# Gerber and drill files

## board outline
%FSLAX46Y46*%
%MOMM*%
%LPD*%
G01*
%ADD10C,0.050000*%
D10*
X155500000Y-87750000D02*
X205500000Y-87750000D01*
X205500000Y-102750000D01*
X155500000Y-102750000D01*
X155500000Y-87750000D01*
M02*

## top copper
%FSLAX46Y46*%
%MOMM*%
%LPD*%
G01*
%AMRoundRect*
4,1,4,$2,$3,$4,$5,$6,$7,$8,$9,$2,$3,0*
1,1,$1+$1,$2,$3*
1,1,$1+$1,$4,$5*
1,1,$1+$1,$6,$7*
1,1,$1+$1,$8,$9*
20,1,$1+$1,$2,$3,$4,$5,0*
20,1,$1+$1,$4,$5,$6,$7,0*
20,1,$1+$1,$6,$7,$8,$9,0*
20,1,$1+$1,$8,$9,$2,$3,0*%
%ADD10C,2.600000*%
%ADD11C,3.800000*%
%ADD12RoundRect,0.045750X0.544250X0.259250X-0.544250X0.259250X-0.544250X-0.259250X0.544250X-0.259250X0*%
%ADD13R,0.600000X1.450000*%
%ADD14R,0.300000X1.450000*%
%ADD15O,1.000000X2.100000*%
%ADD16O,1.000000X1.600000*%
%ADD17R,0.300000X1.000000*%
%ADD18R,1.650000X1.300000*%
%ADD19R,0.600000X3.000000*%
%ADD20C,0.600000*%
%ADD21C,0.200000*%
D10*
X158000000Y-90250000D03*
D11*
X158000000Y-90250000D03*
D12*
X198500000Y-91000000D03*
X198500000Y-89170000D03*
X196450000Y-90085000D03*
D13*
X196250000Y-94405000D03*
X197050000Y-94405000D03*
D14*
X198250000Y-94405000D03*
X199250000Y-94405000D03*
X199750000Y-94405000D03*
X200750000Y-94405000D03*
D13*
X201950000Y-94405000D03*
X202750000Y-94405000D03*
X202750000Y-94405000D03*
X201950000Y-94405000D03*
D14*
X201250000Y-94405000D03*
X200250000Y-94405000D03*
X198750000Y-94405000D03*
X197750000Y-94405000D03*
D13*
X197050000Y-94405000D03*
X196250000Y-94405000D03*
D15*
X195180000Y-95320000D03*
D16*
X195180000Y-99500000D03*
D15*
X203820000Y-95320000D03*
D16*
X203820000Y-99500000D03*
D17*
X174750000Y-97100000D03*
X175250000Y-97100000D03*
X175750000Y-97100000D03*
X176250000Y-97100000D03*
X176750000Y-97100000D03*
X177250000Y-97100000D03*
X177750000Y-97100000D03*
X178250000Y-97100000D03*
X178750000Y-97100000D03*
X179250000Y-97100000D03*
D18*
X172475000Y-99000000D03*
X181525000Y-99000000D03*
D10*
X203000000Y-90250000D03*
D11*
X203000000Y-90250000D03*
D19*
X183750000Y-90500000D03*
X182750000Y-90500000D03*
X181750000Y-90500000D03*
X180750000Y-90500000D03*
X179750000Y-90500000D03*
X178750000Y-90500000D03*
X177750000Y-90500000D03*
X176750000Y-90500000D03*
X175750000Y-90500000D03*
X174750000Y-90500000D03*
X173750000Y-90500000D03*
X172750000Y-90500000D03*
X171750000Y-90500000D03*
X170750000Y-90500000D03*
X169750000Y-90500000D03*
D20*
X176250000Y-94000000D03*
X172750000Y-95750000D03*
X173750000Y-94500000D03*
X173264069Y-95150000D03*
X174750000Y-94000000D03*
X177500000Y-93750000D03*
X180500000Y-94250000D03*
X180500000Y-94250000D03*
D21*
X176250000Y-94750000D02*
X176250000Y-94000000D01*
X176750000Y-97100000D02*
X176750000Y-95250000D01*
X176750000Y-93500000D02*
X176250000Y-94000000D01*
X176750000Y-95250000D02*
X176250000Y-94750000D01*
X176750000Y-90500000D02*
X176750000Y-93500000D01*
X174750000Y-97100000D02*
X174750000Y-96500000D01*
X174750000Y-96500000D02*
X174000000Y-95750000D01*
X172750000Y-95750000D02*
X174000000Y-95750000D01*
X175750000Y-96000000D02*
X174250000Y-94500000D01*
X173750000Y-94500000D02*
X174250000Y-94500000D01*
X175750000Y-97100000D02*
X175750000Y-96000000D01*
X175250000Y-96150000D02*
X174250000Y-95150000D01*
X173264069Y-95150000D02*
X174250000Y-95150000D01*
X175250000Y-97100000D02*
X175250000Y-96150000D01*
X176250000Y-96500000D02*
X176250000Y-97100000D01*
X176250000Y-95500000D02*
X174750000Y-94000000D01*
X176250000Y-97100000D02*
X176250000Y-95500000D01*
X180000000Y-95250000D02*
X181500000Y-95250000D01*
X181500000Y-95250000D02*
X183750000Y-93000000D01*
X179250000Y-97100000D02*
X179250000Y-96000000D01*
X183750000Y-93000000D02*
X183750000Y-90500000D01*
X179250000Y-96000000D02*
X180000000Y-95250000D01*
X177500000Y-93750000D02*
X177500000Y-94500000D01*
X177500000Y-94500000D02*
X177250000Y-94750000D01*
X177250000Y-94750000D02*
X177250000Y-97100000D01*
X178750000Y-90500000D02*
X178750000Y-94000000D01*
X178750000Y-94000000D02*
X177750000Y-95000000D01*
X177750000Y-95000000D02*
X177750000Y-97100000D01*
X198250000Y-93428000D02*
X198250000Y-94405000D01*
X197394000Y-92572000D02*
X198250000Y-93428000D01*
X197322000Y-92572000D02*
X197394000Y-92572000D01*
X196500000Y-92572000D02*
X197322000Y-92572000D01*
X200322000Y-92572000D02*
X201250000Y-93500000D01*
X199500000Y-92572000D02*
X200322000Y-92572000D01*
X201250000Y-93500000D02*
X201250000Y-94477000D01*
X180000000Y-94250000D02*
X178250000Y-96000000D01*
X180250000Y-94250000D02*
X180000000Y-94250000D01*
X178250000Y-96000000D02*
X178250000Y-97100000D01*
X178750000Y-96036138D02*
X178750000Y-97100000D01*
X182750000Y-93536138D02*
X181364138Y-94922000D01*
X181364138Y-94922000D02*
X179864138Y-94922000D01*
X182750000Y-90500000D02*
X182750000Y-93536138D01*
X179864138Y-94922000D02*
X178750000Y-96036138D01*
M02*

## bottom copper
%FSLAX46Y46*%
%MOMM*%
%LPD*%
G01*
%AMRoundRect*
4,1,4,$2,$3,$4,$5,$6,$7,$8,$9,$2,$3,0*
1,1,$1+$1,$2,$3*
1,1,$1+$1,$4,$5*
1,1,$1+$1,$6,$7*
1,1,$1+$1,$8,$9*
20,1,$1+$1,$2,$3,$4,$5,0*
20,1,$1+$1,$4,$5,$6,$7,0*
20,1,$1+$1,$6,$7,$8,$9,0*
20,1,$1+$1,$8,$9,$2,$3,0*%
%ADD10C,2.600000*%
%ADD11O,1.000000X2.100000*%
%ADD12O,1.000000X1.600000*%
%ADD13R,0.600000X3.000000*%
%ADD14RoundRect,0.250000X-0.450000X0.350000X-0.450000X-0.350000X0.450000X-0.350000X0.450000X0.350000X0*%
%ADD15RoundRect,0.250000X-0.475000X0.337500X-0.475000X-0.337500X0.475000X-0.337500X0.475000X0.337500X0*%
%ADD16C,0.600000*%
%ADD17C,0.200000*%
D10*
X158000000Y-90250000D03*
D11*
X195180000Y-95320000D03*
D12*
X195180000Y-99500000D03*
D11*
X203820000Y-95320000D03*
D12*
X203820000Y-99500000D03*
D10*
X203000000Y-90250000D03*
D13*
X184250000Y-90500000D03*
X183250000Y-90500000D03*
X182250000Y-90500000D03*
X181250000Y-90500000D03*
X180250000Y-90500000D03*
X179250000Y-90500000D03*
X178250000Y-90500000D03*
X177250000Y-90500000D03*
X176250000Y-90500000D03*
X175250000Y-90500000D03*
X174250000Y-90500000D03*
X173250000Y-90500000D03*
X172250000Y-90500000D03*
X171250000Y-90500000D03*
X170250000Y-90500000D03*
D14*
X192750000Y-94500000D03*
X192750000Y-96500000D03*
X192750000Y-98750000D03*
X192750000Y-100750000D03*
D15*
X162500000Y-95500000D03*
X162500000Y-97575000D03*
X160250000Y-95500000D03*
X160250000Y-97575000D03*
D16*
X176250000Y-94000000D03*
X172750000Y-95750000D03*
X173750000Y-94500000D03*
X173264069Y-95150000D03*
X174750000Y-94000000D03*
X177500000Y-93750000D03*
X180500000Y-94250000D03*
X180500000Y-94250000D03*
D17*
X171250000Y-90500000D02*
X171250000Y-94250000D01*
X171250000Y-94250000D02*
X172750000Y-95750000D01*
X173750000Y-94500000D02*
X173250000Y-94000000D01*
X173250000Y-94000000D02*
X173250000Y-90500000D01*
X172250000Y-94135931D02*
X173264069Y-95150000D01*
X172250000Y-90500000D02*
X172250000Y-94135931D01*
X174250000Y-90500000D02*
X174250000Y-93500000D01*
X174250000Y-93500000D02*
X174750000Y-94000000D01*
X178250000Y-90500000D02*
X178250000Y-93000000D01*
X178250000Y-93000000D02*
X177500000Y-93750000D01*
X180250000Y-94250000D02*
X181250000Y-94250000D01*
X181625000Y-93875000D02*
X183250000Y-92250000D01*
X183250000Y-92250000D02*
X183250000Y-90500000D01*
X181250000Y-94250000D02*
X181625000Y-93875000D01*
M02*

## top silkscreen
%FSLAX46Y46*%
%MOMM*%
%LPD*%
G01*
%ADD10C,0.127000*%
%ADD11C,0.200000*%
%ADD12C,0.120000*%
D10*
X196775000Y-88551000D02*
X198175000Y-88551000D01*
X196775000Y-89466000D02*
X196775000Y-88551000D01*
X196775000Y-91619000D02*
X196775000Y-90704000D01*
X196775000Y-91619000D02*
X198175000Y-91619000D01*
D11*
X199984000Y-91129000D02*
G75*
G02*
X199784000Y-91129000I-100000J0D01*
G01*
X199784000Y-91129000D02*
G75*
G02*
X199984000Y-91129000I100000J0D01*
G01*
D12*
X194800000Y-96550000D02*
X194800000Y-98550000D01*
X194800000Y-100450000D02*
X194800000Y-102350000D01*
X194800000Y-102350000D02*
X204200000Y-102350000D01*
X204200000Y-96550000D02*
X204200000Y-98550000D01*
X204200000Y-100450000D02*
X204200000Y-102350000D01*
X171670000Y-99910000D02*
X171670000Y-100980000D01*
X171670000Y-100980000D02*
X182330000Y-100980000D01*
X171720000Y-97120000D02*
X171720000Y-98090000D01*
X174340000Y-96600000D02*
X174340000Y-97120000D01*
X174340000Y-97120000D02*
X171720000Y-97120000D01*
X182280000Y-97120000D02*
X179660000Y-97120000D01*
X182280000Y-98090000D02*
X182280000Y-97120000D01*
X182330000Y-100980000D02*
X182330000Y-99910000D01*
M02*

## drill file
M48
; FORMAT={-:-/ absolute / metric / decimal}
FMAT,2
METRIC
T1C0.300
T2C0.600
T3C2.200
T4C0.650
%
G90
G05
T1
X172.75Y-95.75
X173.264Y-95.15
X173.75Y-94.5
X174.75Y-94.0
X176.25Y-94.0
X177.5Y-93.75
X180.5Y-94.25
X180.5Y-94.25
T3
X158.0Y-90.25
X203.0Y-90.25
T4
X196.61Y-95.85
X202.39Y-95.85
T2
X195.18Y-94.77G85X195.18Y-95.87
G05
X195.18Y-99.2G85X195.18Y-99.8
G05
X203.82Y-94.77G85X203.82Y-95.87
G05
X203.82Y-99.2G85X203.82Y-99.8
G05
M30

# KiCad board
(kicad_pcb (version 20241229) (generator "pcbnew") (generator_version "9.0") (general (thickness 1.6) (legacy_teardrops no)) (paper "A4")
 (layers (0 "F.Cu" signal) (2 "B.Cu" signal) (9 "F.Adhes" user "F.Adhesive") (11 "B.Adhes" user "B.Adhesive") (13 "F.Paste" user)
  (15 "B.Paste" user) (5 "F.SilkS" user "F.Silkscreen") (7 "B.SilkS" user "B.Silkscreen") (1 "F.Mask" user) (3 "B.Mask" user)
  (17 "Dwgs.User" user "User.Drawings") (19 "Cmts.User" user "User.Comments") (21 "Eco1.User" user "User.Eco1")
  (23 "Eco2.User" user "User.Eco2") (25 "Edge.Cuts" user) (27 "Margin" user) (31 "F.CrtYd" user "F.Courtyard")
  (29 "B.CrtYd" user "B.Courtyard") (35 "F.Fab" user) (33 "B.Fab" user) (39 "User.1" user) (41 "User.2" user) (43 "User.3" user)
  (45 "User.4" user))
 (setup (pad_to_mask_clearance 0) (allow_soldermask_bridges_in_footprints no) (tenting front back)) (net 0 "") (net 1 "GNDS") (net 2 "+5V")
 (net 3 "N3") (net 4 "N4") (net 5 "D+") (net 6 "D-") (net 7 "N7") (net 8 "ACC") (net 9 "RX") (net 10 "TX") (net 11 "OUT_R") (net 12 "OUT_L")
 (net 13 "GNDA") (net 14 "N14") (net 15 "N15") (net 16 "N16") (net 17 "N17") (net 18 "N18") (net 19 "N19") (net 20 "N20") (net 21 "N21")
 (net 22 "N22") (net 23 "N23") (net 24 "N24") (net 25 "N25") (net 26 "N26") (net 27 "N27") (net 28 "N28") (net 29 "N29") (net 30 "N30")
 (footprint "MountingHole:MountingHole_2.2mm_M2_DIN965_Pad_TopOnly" (layer "F.Cu") (at 158 90.25)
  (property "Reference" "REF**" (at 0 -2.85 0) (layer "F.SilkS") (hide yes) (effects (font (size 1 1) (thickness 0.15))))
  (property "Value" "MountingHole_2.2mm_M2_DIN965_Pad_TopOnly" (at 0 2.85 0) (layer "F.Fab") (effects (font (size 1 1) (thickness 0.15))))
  (pad "1" thru_hole circle (at 0 0) (size 2.6 2.6) (drill 2.2) (layers "*.Cu" "*.Mask") (remove_unused_layers no) (zone_connect 2))
  (pad "1" connect circle (at 0 0) (size 3.8 3.8) (layers "F.Cu" "F.Mask") (zone_connect 2)))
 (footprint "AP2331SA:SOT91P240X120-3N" (layer "F.Cu") (at 197.475 90.085 180)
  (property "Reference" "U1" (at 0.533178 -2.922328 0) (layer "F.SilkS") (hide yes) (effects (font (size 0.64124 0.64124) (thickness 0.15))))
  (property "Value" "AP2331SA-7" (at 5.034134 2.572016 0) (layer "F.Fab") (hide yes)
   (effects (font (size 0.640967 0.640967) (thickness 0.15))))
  (fp_line (start 0.7 1.534) (end -0.7 1.534) (stroke (width 0.127) (type solid)) (layer "F.SilkS"))
  (fp_line (start 0.7 0.619) (end 0.7 1.534) (stroke (width 0.127) (type solid)) (layer "F.SilkS"))
  (fp_line (start 0.7 -1.534) (end 0.7 -0.619) (stroke (width 0.127) (type solid)) (layer "F.SilkS"))
  (fp_line (start 0.7 -1.534) (end -0.7 -1.534) (stroke (width 0.127) (type solid)) (layer "F.SilkS"))
  (fp_circle (center -2.409 -1.044) (end -2.309 -1.044) (stroke (width 0.2) (type solid)) (fill no) (layer "F.SilkS"))
  (pad "1" smd roundrect (at -1.025 -0.915 180) (size 1.18 0.61) (layers "F.Cu" "F.Mask" "F.Paste") (roundrect_rratio 0.075) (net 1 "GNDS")
   (solder_mask_margin 0.102))
  (pad "2" smd roundrect (at -1.025 0.915 180) (size 1.18 0.61) (layers "F.Cu" "F.Mask" "F.Paste") (roundrect_rratio 0.075) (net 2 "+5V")
   (solder_mask_margin 0.102))
  (pad "3" smd roundrect (at 1.025 0 180) (size 1.18 0.61) (layers "F.Cu" "F.Mask" "F.Paste") (roundrect_rratio 0.075) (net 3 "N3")
   (solder_mask_margin 0.102)))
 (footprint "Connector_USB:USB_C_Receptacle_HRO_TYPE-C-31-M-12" (layer "F.Cu") (at 199.5 98.45)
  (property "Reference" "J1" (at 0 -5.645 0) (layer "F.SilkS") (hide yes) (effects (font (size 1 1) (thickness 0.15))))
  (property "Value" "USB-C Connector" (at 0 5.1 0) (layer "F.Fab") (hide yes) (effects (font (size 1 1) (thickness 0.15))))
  (fp_line (start -4.7 -1.9) (end -4.7 0.1) (stroke (width 0.12) (type solid)) (layer "F.SilkS"))
  (fp_line (start -4.7 2) (end -4.7 3.9) (stroke (width 0.12) (type solid)) (layer "F.SilkS"))
  (fp_line (start -4.7 3.9) (end 4.7 3.9) (stroke (width 0.12) (type solid)) (layer "F.SilkS"))
  (fp_line (start 4.7 -1.9) (end 4.7 0.1) (stroke (width 0.12) (type solid)) (layer "F.SilkS"))
  (fp_line (start 4.7 2) (end 4.7 3.9) (stroke (width 0.12) (type solid)) (layer "F.SilkS"))
  (pad "" np_thru_hole circle (at -2.89 -2.6) (size 0.65 0.65) (drill 0.65) (layers "*.Cu" "*.Mask"))
  (pad "" np_thru_hole circle (at 2.89 -2.6) (size 0.65 0.65) (drill 0.65) (layers "*.Cu" "*.Mask"))
  (pad "A1" smd rect (at -3.25 -4.045) (size 0.6 1.45) (layers "F.Cu" "F.Mask" "F.Paste") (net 1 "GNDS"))
  (pad "A4" smd rect (at -2.45 -4.045) (size 0.6 1.45) (layers "F.Cu" "F.Mask" "F.Paste") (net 3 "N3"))
  (pad "A5" smd rect (at -1.25 -4.045) (size 0.3 1.45) (layers "F.Cu" "F.Mask" "F.Paste") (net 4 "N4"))
  (pad "A6" smd rect (at -0.25 -4.045) (size 0.3 1.45) (layers "F.Cu" "F.Mask" "F.Paste") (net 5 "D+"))
  (pad "A7" smd rect (at 0.25 -4.045) (size 0.3 1.45) (layers "F.Cu" "F.Mask" "F.Paste") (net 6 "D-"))
  (pad "A8" smd rect (at 1.25 -4.045) (size 0.3 1.45) (layers "F.Cu" "F.Mask" "F.Paste"))
  (pad "A9" smd rect (at 2.45 -4.045) (size 0.6 1.45) (layers "F.Cu" "F.Mask" "F.Paste") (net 3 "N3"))
  (pad "A12" smd rect (at 3.25 -4.045) (size 0.6 1.45) (layers "F.Cu" "F.Mask" "F.Paste") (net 1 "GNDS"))
  (pad "B1" smd rect (at 3.25 -4.045) (size 0.6 1.45) (layers "F.Cu" "F.Mask" "F.Paste") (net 1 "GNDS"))
  (pad "B4" smd rect (at 2.45 -4.045) (size 0.6 1.45) (layers "F.Cu" "F.Mask" "F.Paste") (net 3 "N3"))
  (pad "B5" smd rect (at 1.75 -4.045) (size 0.3 1.45) (layers "F.Cu" "F.Mask" "F.Paste") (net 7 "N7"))
  (pad "B6" smd rect (at 0.75 -4.045) (size 0.3 1.45) (layers "F.Cu" "F.Mask" "F.Paste") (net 5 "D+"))
  (pad "B7" smd rect (at -0.75 -4.045) (size 0.3 1.45) (layers "F.Cu" "F.Mask" "F.Paste") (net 6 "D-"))
  (pad "B8" smd rect (at -1.75 -4.045) (size 0.3 1.45) (layers "F.Cu" "F.Mask" "F.Paste"))
  (pad "B9" smd rect (at -2.45 -4.045) (size 0.6 1.45) (layers "F.Cu" "F.Mask" "F.Paste") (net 3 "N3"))
  (pad "B12" smd rect (at -3.25 -4.045) (size 0.6 1.45) (layers "F.Cu" "F.Mask" "F.Paste") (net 1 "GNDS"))
  (pad "S1" thru_hole oval (at -4.32 -3.13) (size 1 2.1) (drill oval 0.6 1.7) (layers "*.Cu" "*.Mask") (remove_unused_layers no)
   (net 1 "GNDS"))
  (pad "S1" thru_hole oval (at -4.32 1.05) (size 1 1.6) (drill oval 0.6 1.2) (layers "*.Cu" "*.Mask") (remove_unused_layers no)
   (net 1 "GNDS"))
  (pad "S1" thru_hole oval (at 4.32 -3.13) (size 1 2.1) (drill oval 0.6 1.7) (layers "*.Cu" "*.Mask") (remove_unused_layers no)
   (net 1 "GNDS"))
  (pad "S1" thru_hole oval (at 4.32 1.05) (size 1 1.6) (drill oval 0.6 1.2) (layers "*.Cu" "*.Mask") (remove_unused_layers no)
   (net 1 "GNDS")))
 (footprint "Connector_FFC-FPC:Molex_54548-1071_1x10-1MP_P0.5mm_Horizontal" (layer "F.Cu") (at 177 98.125)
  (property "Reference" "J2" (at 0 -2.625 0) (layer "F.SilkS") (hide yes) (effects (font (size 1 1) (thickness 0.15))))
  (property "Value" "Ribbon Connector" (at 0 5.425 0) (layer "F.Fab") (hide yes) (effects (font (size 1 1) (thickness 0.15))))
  (fp_line (start -5.33 1.785) (end -5.33 2.855) (stroke (width 0.12) (type solid)) (layer "F.SilkS"))
  (fp_line (start -5.33 2.855) (end 5.33 2.855) (stroke (width 0.12) (type solid)) (layer "F.SilkS"))
  (fp_line (start -5.28 -1.005) (end -5.28 -0.035) (stroke (width 0.12) (type solid)) (layer "F.SilkS"))
  (fp_line (start -2.66 -1.525) (end -2.66 -1.005) (stroke (width 0.12) (type solid)) (layer "F.SilkS"))
  (fp_line (start -2.66 -1.005) (end -5.28 -1.005) (stroke (width 0.12) (type solid)) (layer "F.SilkS"))
  (fp_line (start 5.28 -1.005) (end 2.66 -1.005) (stroke (width 0.12) (type solid)) (layer "F.SilkS"))
  (fp_line (start 5.28 -0.035) (end 5.28 -1.005) (stroke (width 0.12) (type solid)) (layer "F.SilkS"))
  (fp_line (start 5.33 2.855) (end 5.33 1.785) (stroke (width 0.12) (type solid)) (layer "F.SilkS"))
  (pad "1" smd rect (at -2.25 -1.025) (size 0.3 1) (layers "F.Cu" "F.Mask" "F.Paste") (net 5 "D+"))
  (pad "2" smd rect (at -1.75 -1.025) (size 0.3 1) (layers "F.Cu" "F.Mask" "F.Paste") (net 6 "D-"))
  (pad "3" smd rect (at -1.25 -1.025) (size 0.3 1) (layers "F.Cu" "F.Mask" "F.Paste") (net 2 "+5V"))
  (pad "4" smd rect (at -0.75 -1.025) (size 0.3 1) (layers "F.Cu" "F.Mask" "F.Paste") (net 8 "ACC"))
  (pad "5" smd rect (at -0.25 -1.025) (size 0.3 1) (layers "F.Cu" "F.Mask" "F.Paste") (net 1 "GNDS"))
  (pad "6" smd rect (at 0.25 -1.025) (size 0.3 1) (layers "F.Cu" "F.Mask" "F.Paste") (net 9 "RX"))
  (pad "7" smd rect (at 0.75 -1.025) (size 0.3 1) (layers "F.Cu" "F.Mask" "F.Paste") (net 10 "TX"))
  (pad "8" smd rect (at 1.25 -1.025) (size 0.3 1) (layers "F.Cu" "F.Mask" "F.Paste") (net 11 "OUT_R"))
  (pad "9" smd rect (at 1.75 -1.025) (size 0.3 1) (layers "F.Cu" "F.Mask" "F.Paste") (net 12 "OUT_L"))
  (pad "10" smd rect (at 2.25 -1.025) (size 0.3 1) (layers "F.Cu" "F.Mask" "F.Paste") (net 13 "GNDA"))
  (pad "MP" smd rect (at -4.525 0.875) (size 1.65 1.3) (layers "F.Cu" "F.Mask" "F.Paste"))
  (pad "MP" smd rect (at 4.525 0.875) (size 1.65 1.3) (layers "F.Cu" "F.Mask" "F.Paste")))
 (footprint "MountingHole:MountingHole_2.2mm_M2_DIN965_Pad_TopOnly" (layer "F.Cu") (at 203 90.25)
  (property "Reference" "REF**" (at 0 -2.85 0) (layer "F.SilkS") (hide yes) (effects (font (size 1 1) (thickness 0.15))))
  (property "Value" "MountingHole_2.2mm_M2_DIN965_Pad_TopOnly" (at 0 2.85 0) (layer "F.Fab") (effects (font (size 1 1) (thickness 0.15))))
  (pad "1" thru_hole circle (at 0 0) (size 2.6 2.6) (drill 2.2) (layers "*.Cu" "*.Mask") (remove_unused_layers no) (zone_connect 2))
  (pad "1" connect circle (at 0 0) (size 3.8 3.8) (layers "F.Cu" "F.Mask") (zone_connect 2)))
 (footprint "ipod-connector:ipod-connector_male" (layer "F.Cu") (at 176.75 90.5)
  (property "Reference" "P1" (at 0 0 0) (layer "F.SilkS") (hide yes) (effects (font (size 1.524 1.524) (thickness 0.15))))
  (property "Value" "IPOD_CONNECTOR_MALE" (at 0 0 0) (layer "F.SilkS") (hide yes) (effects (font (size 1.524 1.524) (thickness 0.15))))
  (pad "1" smd rect (at 7.5 0) (size 0.6 3) (layers "B.Cu" "B.Mask" "B.Paste") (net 13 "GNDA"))
  (pad "2" smd rect (at 7 0) (size 0.6 3) (layers "F.Cu" "F.Mask" "F.Paste") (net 13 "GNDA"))
  (pad "3" smd rect (at 6.5 0) (size 0.6 3) (layers "B.Cu" "B.Mask" "B.Paste") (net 11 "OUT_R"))
  (pad "4" smd rect (at 6 0) (size 0.6 3) (layers "F.Cu" "F.Mask" "F.Paste") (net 12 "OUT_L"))
  (pad "5" smd rect (at 5.5 0) (size 0.6 3) (layers "B.Cu" "B.Mask" "B.Paste") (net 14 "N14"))
  (pad "6" smd rect (at 5 0) (size 0.6 3) (layers "F.Cu" "F.Mask" "F.Paste") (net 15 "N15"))
  (pad "7" smd rect (at 4.5 0) (size 0.6 3) (layers "B.Cu" "B.Mask" "B.Paste") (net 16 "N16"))
  (pad "8" smd rect (at 4 0) (size 0.6 3) (layers "F.Cu" "F.Mask" "F.Paste") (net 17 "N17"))
  (pad "9" smd rect (at 3.5 0) (size 0.6 3) (layers "B.Cu" "B.Mask" "B.Paste") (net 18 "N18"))
  (pad "10" smd rect (at 3 0) (size 0.6 3) (layers "F.Cu" "F.Mask" "F.Paste") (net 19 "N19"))
  (pad "11" smd rect (at 2.5 0) (size 0.6 3) (layers "B.Cu" "B.Mask" "B.Paste") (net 1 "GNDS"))
  (pad "12" smd rect (at 2 0) (size 0.6 3) (layers "F.Cu" "F.Mask" "F.Paste") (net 10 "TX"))
  (pad "13" smd rect (at 1.5 0) (size 0.6 3) (layers "B.Cu" "B.Mask" "B.Paste") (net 9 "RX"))
  (pad "14" smd rect (at 1 0) (size 0.6 3) (layers "F.Cu" "F.Mask" "F.Paste") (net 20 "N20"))
  (pad "15" smd rect (at 0.5 0) (size 0.6 3) (layers "B.Cu" "B.Mask" "B.Paste") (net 1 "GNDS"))
  (pad "16" smd rect (at 0 0) (size 0.6 3) (layers "F.Cu" "F.Mask" "F.Paste") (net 1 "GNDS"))
  (pad "17" smd rect (at -0.5 0) (size 0.6 3) (layers "B.Cu" "B.Mask" "B.Paste") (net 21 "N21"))
  (pad "18" smd rect (at -1 0) (size 0.6 3) (layers "F.Cu" "F.Mask" "F.Paste") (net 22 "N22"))
  (pad "19" smd rect (at -1.5 0) (size 0.6 3) (layers "B.Cu" "B.Mask" "B.Paste") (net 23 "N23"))
  (pad "20" smd rect (at -2 0) (size 0.6 3) (layers "F.Cu" "F.Mask" "F.Paste") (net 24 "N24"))
  (pad "21" smd rect (at -2.5 0) (size 0.6 3) (layers "B.Cu" "B.Mask" "B.Paste") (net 8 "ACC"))
  (pad "22" smd rect (at -3 0) (size 0.6 3) (layers "F.Cu" "F.Mask" "F.Paste") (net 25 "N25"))
  (pad "23" smd rect (at -3.5 0) (size 0.6 3) (layers "B.Cu" "B.Mask" "B.Paste") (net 2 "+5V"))
  (pad "24" smd rect (at -4 0) (size 0.6 3) (layers "F.Cu" "F.Mask" "F.Paste") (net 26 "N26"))
  (pad "25" smd rect (at -4.5 0) (size 0.6 3) (layers "B.Cu" "B.Mask" "B.Paste") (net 6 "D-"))
  (pad "26" smd rect (at -5 0) (size 0.6 3) (layers "F.Cu" "F.Mask" "F.Paste") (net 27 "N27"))
  (pad "27" smd rect (at -5.5 0) (size 0.6 3) (layers "B.Cu" "B.Mask" "B.Paste") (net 5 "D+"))
  (pad "28" smd rect (at -6 0) (size 0.6 3) (layers "F.Cu" "F.Mask" "F.Paste") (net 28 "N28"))
  (pad "29" smd rect (at -6.5 0) (size 0.6 3) (layers "B.Cu" "B.Mask" "B.Paste") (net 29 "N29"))
  (pad "30" smd rect (at -7 0) (size 0.6 3) (layers "F.Cu" "F.Mask" "F.Paste") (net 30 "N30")))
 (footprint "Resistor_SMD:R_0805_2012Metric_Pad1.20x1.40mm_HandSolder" (layer "B.Cu") (at 192.75 95.5 -90)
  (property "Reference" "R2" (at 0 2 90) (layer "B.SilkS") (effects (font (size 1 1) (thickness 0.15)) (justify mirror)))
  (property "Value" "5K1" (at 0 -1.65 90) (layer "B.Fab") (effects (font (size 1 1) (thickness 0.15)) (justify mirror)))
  (pad "1" smd roundrect (at -1 0 270) (size 1.2 1.4) (layers "B.Cu" "B.Mask" "B.Paste") (roundrect_rratio 0.208333) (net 4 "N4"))
  (pad "2" smd roundrect (at 1 0 270) (size 1.2 1.4) (layers "B.Cu" "B.Mask" "B.Paste") (roundrect_rratio 0.208333) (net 1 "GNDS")))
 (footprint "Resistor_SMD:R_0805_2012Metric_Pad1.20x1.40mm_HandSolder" (layer "B.Cu") (at 192.75 99.75 -90)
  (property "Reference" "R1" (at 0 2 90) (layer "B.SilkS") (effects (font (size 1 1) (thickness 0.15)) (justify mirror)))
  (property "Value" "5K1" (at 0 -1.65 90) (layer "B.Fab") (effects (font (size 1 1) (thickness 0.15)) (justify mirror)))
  (pad "1" smd roundrect (at -1 0 270) (size 1.2 1.4) (layers "B.Cu" "B.Mask" "B.Paste") (roundrect_rratio 0.208333) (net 7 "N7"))
  (pad "2" smd roundrect (at 1 0 270) (size 1.2 1.4) (layers "B.Cu" "B.Mask" "B.Paste") (roundrect_rratio 0.208333) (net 1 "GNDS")))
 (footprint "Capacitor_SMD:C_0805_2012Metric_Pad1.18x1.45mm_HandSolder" (layer "B.Cu") (at 162.5 96.5375 -90)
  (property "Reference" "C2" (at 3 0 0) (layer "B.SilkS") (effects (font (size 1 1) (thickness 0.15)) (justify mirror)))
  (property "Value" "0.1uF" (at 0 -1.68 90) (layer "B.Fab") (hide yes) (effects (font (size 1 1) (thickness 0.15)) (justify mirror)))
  (pad "1" smd roundrect (at -1.0375 0 270) (size 1.175 1.45) (layers "B.Cu" "B.Mask" "B.Paste") (roundrect_rratio 0.212766) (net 2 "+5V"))
  (pad "2" smd roundrect (at 1.0375 0 270) (size 1.175 1.45) (layers "B.Cu" "B.Mask" "B.Paste") (roundrect_rratio 0.212766) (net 1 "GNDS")))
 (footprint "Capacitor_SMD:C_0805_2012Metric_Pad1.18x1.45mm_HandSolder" (layer "B.Cu") (at 160.25 96.5375 -90)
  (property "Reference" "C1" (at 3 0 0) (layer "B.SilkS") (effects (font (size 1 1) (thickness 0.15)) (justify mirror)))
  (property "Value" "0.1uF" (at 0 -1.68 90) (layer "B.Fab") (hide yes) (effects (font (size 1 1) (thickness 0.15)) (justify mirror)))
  (pad "1" smd roundrect (at -1.0375 0 270) (size 1.175 1.45) (layers "B.Cu" "B.Mask" "B.Paste") (roundrect_rratio 0.212766) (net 3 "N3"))
  (pad "2" smd roundrect (at 1.0375 0 270) (size 1.175 1.45) (layers "B.Cu" "B.Mask" "B.Paste") (roundrect_rratio 0.212766) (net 1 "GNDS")))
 (gr_rect (start 155.5 87.75) (end 205.5 102.75) (stroke (width 0.05) (type default)) (fill no) (layer "Edge.Cuts"))
 (segment (start 176.25 94.75) (end 176.25 94) (width 0.2) (layer "F.Cu") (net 1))
 (segment (start 176.75 97.1) (end 176.75 95.25) (width 0.2) (layer "F.Cu") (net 1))
 (segment (start 176.75 93.5) (end 176.25 94) (width 0.2) (layer "F.Cu") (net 1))
 (segment (start 176.75 95.25) (end 176.25 94.75) (width 0.2) (layer "F.Cu") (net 1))
 (segment (start 176.75 90.5) (end 176.75 93.5) (width 0.2) (layer "F.Cu") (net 1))
 (via (at 176.25 94) (size 0.6) (drill 0.3) (layers "F.Cu" "B.Cu") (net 1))
 (segment (start 174.75 97.1) (end 174.75 96.5) (width 0.2) (layer "F.Cu") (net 5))
 (segment (start 174.75 96.5) (end 174 95.75) (width 0.2) (layer "F.Cu") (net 5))
 (segment (start 172.75 95.75) (end 174 95.75) (width 0.2) (layer "F.Cu") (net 5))
 (via (at 172.75 95.75) (size 0.6) (drill 0.3) (layers "F.Cu" "B.Cu") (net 5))
 (segment (start 171.25 90.5) (end 171.25 94.25) (width 0.2) (layer "B.Cu") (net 5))
 (segment (start 171.25 94.25) (end 172.75 95.75) (width 0.2) (layer "B.Cu") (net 5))
 (segment (start 175.75 96) (end 174.25 94.5) (width 0.2) (layer "F.Cu") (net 2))
 (segment (start 173.75 94.5) (end 174.25 94.5) (width 0.2) (layer "F.Cu") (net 2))
 (segment (start 175.75 97.1) (end 175.75 96) (width 0.2) (layer "F.Cu") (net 2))
 (via (at 173.75 94.5) (size 0.6) (drill 0.3) (layers "F.Cu" "B.Cu") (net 2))
 (segment (start 173.75 94.5) (end 173.25 94) (width 0.2) (layer "B.Cu") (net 2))
 (segment (start 173.25 94) (end 173.25 90.5) (width 0.2) (layer "B.Cu") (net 2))
 (segment (start 175.25 96.15) (end 174.25 95.15) (width 0.2) (layer "F.Cu") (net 6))
 (segment (start 173.264069 95.15) (end 174.25 95.15) (width 0.2) (layer "F.Cu") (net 6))
 (segment (start 175.25 97.1) (end 175.25 96.15) (width 0.2) (layer "F.Cu") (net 6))
 (via (at 173.264069 95.15) (size 0.6) (drill 0.3) (layers "F.Cu" "B.Cu") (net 6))
 (segment (start 172.25 94.135931) (end 173.264069 95.15) (width 0.2) (layer "B.Cu") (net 6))
 (segment (start 172.25 90.5) (end 172.25 94.135931) (width 0.2) (layer "B.Cu") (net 6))
 (segment (start 176.25 96.5) (end 176.25 97.1) (width 0.2) (layer "F.Cu") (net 8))
 (segment (start 176.25 95.5) (end 174.75 94) (width 0.2) (layer "F.Cu") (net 8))
 (segment (start 176.25 97.1) (end 176.25 95.5) (width 0.2) (layer "F.Cu") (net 8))
 (via (at 174.75 94) (size 0.6) (drill 0.3) (layers "F.Cu" "B.Cu") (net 8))
 (segment (start 174.25 90.5) (end 174.25 93.5) (width 0.2) (layer "B.Cu") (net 8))
 (segment (start 174.25 93.5) (end 174.75 94) (width 0.2) (layer "B.Cu") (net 8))
 (segment (start 180 95.25) (end 181.5 95.25) (width 0.2) (layer "F.Cu") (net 13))
 (segment (start 181.5 95.25) (end 183.75 93) (width 0.2) (layer "F.Cu") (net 13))
 (segment (start 179.25 97.1) (end 179.25 96) (width 0.2) (layer "F.Cu") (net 13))
 (segment (start 183.75 93) (end 183.75 90.5) (width 0.2) (layer "F.Cu") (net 13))
 (segment (start 179.25 96) (end 180 95.25) (width 0.2) (layer "F.Cu") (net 13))
 (segment (start 177.5 93.75) (end 177.5 94.5) (width 0.2) (layer "F.Cu") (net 9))
 (segment (start 177.5 94.5) (end 177.25 94.75) (width 0.2) (layer "F.Cu") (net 9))
 (segment (start 177.25 94.75) (end 177.25 97.1) (width 0.2) (layer "F.Cu") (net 9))
 (via (at 177.5 93.75) (size 0.6) (drill 0.3) (layers "F.Cu" "B.Cu") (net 9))
 (segment (start 178.25 90.5) (end 178.25 93) (width 0.2) (layer "B.Cu") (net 9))
 (segment (start 178.25 93) (end 177.5 93.75) (width 0.2) (layer "B.Cu") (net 9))
 (segment (start 178.75 90.5) (end 178.75 94) (width 0.2) (layer "F.Cu") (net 10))
 (segment (start 178.75 94) (end 177.75 95) (width 0.2) (layer "F.Cu") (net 10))
 (segment (start 177.75 95) (end 177.75 97.1) (width 0.2) (layer "F.Cu") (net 10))
 (segment (start 198.25 93.428) (end 198.25 94.405) (width 0.2) (layer "F.Cu") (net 4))
 (segment (start 197.394 92.572) (end 198.25 93.428) (width 0.2) (layer "F.Cu") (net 4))
 (segment (start 197.322 92.572) (end 197.394 92.572) (width 0.2) (layer "F.Cu") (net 4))
 (segment (start 196.5 92.572) (end 197.322 92.572) (width 0.2) (layer "F.Cu") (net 4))
 (segment (start 200.322 92.572) (end 201.25 93.5) (width 0.2) (layer "F.Cu") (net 7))
 (segment (start 199.5 92.572) (end 200.322 92.572) (width 0.2) (layer "F.Cu") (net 7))
 (segment (start 201.25 93.5) (end 201.25 94.477) (width 0.2) (layer "F.Cu") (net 7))
 (segment (start 180 94.25) (end 178.25 96) (width 0.2) (layer "F.Cu") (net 11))
 (segment (start 180.25 94.25) (end 180 94.25) (width 0.2) (layer "F.Cu") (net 11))
 (segment (start 178.25 96) (end 178.25 97.1) (width 0.2) (layer "F.Cu") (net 11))
 (via (at 180.5 94.25) (size 0.6) (drill 0.3) (layers "F.Cu" "B.Cu") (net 11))
 (via (at 180.5 94.25) (size 0.6) (drill 0.3) (layers "F.Cu" "B.Cu") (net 11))
 (segment (start 180.25 94.25) (end 181.25 94.25) (width 0.2) (layer "B.Cu") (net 11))
 (segment (start 181.625 93.875) (end 183.25 92.25) (width 0.2) (layer "B.Cu") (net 11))
 (segment (start 183.25 92.25) (end 183.25 90.5) (width 0.2) (layer "B.Cu") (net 11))
 (segment (start 181.25 94.25) (end 181.625 93.875) (width 0.2) (layer "B.Cu") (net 11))
 (segment (start 178.75 96.036138) (end 178.75 97.1) (width 0.2) (layer "F.Cu") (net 12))
 (segment (start 182.75 93.536138) (end 181.364138 94.922) (width 0.2) (layer "F.Cu") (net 12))
 (segment (start 181.364138 94.922) (end 179.864138 94.922) (width 0.2) (layer "F.Cu") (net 12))
 (segment (start 182.75 90.5) (end 182.75 93.536138) (width 0.2) (layer "F.Cu") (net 12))
 (segment (start 179.864138 94.922) (end 178.75 96.036138) (width 0.2) (layer "F.Cu") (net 12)))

